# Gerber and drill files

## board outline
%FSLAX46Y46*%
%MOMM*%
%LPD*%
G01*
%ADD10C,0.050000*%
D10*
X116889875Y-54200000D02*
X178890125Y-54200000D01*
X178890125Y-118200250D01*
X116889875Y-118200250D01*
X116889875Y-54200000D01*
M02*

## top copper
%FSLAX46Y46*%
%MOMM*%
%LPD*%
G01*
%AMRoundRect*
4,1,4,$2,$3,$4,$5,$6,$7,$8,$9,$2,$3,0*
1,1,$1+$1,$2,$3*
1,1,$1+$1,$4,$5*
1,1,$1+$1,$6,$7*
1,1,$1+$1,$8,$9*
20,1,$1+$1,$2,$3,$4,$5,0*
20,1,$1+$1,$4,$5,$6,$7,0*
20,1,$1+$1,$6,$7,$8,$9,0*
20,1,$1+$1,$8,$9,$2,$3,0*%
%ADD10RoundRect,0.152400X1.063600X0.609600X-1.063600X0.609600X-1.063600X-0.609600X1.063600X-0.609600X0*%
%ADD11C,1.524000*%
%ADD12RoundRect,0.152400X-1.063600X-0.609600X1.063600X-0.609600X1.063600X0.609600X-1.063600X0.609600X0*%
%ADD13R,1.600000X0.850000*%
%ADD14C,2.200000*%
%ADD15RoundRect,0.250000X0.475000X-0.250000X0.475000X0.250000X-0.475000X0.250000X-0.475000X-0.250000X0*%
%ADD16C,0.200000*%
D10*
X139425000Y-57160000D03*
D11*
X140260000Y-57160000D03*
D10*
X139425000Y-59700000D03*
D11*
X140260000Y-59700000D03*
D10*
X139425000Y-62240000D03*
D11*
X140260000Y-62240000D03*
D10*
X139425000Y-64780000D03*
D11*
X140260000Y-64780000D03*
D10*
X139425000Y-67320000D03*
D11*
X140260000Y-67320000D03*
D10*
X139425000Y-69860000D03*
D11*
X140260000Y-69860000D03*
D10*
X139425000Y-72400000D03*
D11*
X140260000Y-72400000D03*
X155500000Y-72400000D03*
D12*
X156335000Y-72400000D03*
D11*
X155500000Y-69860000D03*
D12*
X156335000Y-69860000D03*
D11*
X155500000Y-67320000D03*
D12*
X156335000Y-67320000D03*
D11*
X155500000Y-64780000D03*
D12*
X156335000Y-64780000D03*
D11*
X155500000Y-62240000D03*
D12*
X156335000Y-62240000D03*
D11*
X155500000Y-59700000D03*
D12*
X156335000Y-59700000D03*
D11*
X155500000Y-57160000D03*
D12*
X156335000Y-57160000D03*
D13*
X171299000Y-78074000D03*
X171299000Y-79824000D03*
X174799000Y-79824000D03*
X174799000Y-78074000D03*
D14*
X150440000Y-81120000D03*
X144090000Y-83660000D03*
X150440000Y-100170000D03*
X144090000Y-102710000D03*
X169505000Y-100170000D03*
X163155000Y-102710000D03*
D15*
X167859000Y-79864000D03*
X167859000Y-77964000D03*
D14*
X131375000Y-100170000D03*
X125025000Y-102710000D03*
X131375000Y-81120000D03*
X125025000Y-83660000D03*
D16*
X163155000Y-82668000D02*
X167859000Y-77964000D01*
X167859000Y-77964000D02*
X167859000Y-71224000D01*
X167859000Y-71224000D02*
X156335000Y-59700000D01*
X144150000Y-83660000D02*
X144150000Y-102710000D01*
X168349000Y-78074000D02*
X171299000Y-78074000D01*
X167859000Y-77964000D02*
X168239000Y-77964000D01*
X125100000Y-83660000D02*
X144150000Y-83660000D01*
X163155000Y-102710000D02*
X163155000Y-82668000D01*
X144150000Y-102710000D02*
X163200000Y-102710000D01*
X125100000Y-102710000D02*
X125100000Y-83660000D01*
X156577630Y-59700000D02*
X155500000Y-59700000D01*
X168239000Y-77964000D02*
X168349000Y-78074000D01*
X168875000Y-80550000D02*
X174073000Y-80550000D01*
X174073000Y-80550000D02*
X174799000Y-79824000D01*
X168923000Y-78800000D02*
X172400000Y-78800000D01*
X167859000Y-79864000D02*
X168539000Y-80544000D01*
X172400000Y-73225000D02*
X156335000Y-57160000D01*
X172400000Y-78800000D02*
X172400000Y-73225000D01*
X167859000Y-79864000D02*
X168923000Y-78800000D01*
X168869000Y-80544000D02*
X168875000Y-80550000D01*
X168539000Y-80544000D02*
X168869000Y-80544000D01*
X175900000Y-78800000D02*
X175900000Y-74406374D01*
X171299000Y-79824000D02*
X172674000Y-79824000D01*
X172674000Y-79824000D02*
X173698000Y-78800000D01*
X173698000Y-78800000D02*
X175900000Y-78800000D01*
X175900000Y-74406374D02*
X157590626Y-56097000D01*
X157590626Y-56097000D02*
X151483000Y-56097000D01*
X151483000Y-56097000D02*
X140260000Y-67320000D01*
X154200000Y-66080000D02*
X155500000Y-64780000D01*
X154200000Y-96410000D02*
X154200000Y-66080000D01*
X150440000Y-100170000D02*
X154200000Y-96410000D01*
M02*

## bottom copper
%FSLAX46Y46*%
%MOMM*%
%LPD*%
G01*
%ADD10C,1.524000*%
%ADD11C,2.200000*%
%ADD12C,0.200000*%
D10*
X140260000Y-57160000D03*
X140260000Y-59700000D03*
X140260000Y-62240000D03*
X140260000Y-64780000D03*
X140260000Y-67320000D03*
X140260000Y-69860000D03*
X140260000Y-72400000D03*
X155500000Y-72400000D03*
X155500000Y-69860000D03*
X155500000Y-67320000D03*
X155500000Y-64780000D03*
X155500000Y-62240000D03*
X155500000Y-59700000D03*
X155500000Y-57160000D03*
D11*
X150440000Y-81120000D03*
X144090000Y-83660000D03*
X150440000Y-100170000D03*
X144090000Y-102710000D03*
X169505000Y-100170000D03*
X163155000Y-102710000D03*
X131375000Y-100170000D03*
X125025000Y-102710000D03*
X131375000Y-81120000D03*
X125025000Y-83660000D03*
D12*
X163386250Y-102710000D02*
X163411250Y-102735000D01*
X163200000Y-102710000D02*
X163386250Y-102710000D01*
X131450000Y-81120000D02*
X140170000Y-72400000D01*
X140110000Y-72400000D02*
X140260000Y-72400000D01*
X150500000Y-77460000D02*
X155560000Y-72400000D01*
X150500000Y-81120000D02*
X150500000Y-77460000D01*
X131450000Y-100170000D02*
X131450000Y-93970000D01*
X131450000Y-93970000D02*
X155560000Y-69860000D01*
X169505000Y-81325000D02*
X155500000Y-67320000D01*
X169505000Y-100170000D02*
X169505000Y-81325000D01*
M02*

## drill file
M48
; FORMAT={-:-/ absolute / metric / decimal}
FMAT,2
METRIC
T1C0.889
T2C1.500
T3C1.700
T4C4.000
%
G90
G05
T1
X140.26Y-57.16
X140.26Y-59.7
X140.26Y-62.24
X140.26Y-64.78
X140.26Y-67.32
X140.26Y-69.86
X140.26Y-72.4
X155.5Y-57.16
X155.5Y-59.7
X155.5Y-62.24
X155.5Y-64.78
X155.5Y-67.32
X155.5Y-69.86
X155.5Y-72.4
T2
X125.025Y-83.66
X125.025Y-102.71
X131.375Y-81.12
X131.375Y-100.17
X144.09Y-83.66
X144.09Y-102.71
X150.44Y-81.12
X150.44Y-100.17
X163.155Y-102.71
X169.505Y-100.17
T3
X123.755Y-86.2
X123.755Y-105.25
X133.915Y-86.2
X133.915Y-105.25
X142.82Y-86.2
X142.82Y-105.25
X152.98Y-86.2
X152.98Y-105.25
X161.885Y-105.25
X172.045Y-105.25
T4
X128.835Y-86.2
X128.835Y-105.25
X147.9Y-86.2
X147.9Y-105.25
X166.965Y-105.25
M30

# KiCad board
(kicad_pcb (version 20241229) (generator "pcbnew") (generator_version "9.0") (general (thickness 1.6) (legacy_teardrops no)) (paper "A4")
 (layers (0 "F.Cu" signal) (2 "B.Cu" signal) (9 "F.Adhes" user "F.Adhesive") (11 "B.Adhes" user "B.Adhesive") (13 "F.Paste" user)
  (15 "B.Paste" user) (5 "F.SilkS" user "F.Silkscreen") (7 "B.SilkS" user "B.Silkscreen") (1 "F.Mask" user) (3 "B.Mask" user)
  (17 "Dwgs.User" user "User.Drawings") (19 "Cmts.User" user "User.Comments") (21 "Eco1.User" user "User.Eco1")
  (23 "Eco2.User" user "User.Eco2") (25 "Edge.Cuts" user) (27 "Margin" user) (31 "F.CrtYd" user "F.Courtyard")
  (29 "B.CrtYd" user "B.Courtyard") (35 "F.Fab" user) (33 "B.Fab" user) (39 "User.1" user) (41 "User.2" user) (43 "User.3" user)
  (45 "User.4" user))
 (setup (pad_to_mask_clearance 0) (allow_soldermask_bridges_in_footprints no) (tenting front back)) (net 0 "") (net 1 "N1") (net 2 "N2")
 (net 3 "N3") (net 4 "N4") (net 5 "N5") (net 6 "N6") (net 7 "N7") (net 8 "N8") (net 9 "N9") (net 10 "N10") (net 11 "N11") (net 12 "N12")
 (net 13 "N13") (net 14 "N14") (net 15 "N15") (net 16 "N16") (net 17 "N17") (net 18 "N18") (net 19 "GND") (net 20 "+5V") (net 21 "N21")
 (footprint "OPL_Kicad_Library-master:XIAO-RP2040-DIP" (layer "F.Cu") (at 147.88 64.78)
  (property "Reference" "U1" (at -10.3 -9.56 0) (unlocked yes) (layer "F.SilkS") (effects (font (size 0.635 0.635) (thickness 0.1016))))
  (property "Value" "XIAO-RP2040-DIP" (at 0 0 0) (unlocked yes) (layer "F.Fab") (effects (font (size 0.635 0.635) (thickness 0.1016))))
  (pad "1" smd roundrect (at -8.455 -7.62 180) (size 2.432 1.524) (layers "F.Cu" "F.Mask") (roundrect_rratio 0.1) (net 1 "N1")
   (thermal_bridge_angle 45))
  (pad "1" thru_hole circle (at -7.62 -7.62 180) (size 1.524 1.524) (drill 0.889) (layers "*.Cu" "*.Mask") (remove_unused_layers no)
   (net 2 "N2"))
  (pad "2" smd roundrect (at -8.455 -5.08 180) (size 2.432 1.524) (layers "F.Cu" "F.Mask") (roundrect_rratio 0.1) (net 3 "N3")
   (thermal_bridge_angle 45))
  (pad "2" thru_hole circle (at -7.62 -5.08 180) (size 1.524 1.524) (drill 0.889) (layers "*.Cu" "*.Mask") (remove_unused_layers no)
   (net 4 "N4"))
  (pad "3" smd roundrect (at -8.455 -2.54 180) (size 2.432 1.524) (layers "F.Cu" "F.Mask") (roundrect_rratio 0.1) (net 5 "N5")
   (thermal_bridge_angle 45))
  (pad "3" thru_hole circle (at -7.62 -2.54 180) (size 1.524 1.524) (drill 0.889) (layers "*.Cu" "*.Mask") (remove_unused_layers no)
   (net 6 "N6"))
  (pad "4" smd roundrect (at -8.455 0 180) (size 2.432 1.524) (layers "F.Cu" "F.Mask") (roundrect_rratio 0.1) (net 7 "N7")
   (thermal_bridge_angle 45))
  (pad "4" thru_hole circle (at -7.62 0 180) (size 1.524 1.524) (drill 0.889) (layers "*.Cu" "*.Mask") (remove_unused_layers no)
   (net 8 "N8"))
  (pad "5" smd roundrect (at -8.455 2.54 180) (size 2.432 1.524) (layers "F.Cu" "F.Mask") (roundrect_rratio 0.1) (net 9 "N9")
   (thermal_bridge_angle 45))
  (pad "5" thru_hole circle (at -7.62 2.54 180) (size 1.524 1.524) (drill 0.889) (layers "*.Cu" "*.Mask") (remove_unused_layers no)
   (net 9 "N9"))
  (pad "6" smd roundrect (at -8.455 5.08 180) (size 2.432 1.524) (layers "F.Cu" "F.Mask") (roundrect_rratio 0.1) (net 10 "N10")
   (thermal_bridge_angle 45))
  (pad "6" thru_hole circle (at -7.62 5.08 180) (size 1.524 1.524) (drill 0.889) (layers "*.Cu" "*.Mask") (remove_unused_layers no)
   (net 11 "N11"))
  (pad "7" smd roundrect (at -8.455 7.62 180) (size 2.432 1.524) (layers "F.Cu" "F.Mask") (roundrect_rratio 0.1) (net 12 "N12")
   (thermal_bridge_angle 45))
  (pad "7" thru_hole circle (at -7.62 7.62 180) (size 1.524 1.524) (drill 0.889) (layers "*.Cu" "*.Mask") (remove_unused_layers no)
   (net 12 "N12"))
  (pad "8" thru_hole circle (at 7.62 7.62) (size 1.524 1.524) (drill 0.889) (layers "*.Cu" "*.Mask") (remove_unused_layers no)
   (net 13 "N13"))
  (pad "8" smd roundrect (at 8.455 7.62) (size 2.432 1.524) (layers "F.Cu" "F.Mask") (roundrect_rratio 0.1) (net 13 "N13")
   (thermal_bridge_angle 45))
  (pad "9" thru_hole circle (at 7.62 5.08) (size 1.524 1.524) (drill 0.889) (layers "*.Cu" "*.Mask") (remove_unused_layers no)
   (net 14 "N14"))
  (pad "9" smd roundrect (at 8.455 5.08) (size 2.432 1.524) (layers "F.Cu" "F.Mask") (roundrect_rratio 0.1) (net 14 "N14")
   (thermal_bridge_angle 45))
  (pad "10" thru_hole circle (at 7.62 2.54) (size 1.524 1.524) (drill 0.889) (layers "*.Cu" "*.Mask") (remove_unused_layers no)
   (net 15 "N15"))
  (pad "10" smd roundrect (at 8.455 2.54) (size 2.432 1.524) (layers "F.Cu" "F.Mask") (roundrect_rratio 0.1) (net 15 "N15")
   (thermal_bridge_angle 45))
  (pad "11" thru_hole circle (at 7.62 0) (size 1.524 1.524) (drill 0.889) (layers "*.Cu" "*.Mask") (remove_unused_layers no) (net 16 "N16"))
  (pad "11" smd roundrect (at 8.455 0) (size 2.432 1.524) (layers "F.Cu" "F.Mask") (roundrect_rratio 0.1) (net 16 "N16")
   (thermal_bridge_angle 45))
  (pad "12" thru_hole circle (at 7.62 -2.54) (size 1.524 1.524) (drill 0.889) (layers "*.Cu" "*.Mask") (remove_unused_layers no)
   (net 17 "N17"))
  (pad "12" smd roundrect (at 8.455 -2.54) (size 2.432 1.524) (layers "F.Cu" "F.Mask") (roundrect_rratio 0.1) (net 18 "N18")
   (thermal_bridge_angle 45))
  (pad "13" thru_hole circle (at 7.62 -5.08) (size 1.524 1.524) (drill 0.889) (layers "*.Cu" "*.Mask") (remove_unused_layers no)
   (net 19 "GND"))
  (pad "13" smd roundrect (at 8.455 -5.08) (size 2.432 1.524) (layers "F.Cu" "F.Mask") (roundrect_rratio 0.1) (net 19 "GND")
   (thermal_bridge_angle 45))
  (pad "14" thru_hole circle (at 7.62 -7.62) (size 1.524 1.524) (drill 0.889) (layers "*.Cu" "*.Mask") (remove_unused_layers no)
   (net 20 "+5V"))
  (pad "14" smd roundrect (at 8.455 -7.62) (size 2.432 1.524) (layers "F.Cu" "F.Mask") (roundrect_rratio 0.1) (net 20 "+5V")
   (thermal_bridge_angle 45)))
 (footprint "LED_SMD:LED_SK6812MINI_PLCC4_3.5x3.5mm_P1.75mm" (layer "F.Cu") (at 173.049 78.949)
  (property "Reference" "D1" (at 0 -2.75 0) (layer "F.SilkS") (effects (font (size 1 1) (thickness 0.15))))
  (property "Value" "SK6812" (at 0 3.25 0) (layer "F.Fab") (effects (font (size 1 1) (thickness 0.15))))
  (pad "1" smd rect (at -1.75 -0.875) (size 1.6 0.85) (layers "F.Cu" "F.Mask" "F.Paste") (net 19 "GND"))
  (pad "2" smd rect (at -1.75 0.875) (size 1.6 0.85) (layers "F.Cu" "F.Mask" "F.Paste") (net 9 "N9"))
  (pad "3" smd rect (at 1.75 0.875) (size 1.6 0.85) (layers "F.Cu" "F.Mask" "F.Paste") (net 20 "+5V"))
  (pad "4" smd rect (at 1.75 -0.875) (size 1.6 0.85) (layers "F.Cu" "F.Mask" "F.Paste") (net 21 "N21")))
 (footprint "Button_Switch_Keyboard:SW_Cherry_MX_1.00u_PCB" (layer "F.Cu") (at 150.44 81.12)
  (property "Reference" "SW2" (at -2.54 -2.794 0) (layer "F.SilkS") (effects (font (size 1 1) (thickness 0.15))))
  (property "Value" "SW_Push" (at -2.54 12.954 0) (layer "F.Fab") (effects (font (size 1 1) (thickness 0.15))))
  (pad "" np_thru_hole circle (at -7.62 5.08) (size 1.7 1.7) (drill 1.7) (layers "*.Cu" "*.Mask"))
  (pad "" np_thru_hole circle (at -2.54 5.08) (size 4 4) (drill 4) (layers "*.Cu" "*.Mask"))
  (pad "" np_thru_hole circle (at 2.54 5.08) (size 1.7 1.7) (drill 1.7) (layers "*.Cu" "*.Mask"))
  (pad "1" thru_hole circle (at 0 0) (size 2.2 2.2) (drill 1.5) (layers "*.Cu" "*.Mask") (remove_unused_layers no) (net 13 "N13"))
  (pad "2" thru_hole circle (at -6.35 2.54) (size 2.2 2.2) (drill 1.5) (layers "*.Cu" "*.Mask") (remove_unused_layers no) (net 19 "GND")))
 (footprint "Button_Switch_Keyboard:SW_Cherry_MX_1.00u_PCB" (layer "F.Cu") (at 150.44 100.17)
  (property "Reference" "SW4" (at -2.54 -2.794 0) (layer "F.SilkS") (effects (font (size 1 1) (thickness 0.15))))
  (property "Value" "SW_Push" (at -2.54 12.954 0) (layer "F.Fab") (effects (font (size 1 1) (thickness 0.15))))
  (pad "" np_thru_hole circle (at -7.62 5.08) (size 1.7 1.7) (drill 1.7) (layers "*.Cu" "*.Mask"))
  (pad "" np_thru_hole circle (at -2.54 5.08) (size 4 4) (drill 4) (layers "*.Cu" "*.Mask"))
  (pad "" np_thru_hole circle (at 2.54 5.08) (size 1.7 1.7) (drill 1.7) (layers "*.Cu" "*.Mask"))
  (pad "1" thru_hole circle (at 0 0) (size 2.2 2.2) (drill 1.5) (layers "*.Cu" "*.Mask") (remove_unused_layers no) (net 16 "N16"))
  (pad "2" thru_hole circle (at -6.35 2.54) (size 2.2 2.2) (drill 1.5) (layers "*.Cu" "*.Mask") (remove_unused_layers no) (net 19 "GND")))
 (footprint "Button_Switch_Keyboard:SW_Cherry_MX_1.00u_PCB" (layer "F.Cu") (at 169.505 100.17)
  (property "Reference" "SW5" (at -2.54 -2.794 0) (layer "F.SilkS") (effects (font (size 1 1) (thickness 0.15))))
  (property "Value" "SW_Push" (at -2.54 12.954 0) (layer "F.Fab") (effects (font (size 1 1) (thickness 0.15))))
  (pad "" np_thru_hole circle (at -7.62 5.08) (size 1.7 1.7) (drill 1.7) (layers "*.Cu" "*.Mask"))
  (pad "" np_thru_hole circle (at -2.54 5.08) (size 4 4) (drill 4) (layers "*.Cu" "*.Mask"))
  (pad "" np_thru_hole circle (at 2.54 5.08) (size 1.7 1.7) (drill 1.7) (layers "*.Cu" "*.Mask"))
  (pad "1" thru_hole circle (at 0 0) (size 2.2 2.2) (drill 1.5) (layers "*.Cu" "*.Mask") (remove_unused_layers no) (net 15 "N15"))
  (pad "2" thru_hole circle (at -6.35 2.54) (size 2.2 2.2) (drill 1.5) (layers "*.Cu" "*.Mask") (remove_unused_layers no) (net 19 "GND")))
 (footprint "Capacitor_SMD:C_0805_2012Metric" (layer "F.Cu") (at 167.859 78.914 90)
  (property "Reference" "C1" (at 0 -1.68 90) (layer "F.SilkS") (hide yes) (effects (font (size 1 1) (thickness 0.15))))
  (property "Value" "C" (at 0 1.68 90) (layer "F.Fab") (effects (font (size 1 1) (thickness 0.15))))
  (pad "1" smd roundrect (at -0.95 0 90) (size 1 1.45) (layers "F.Cu" "F.Mask" "F.Paste") (roundrect_rratio 0.25) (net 20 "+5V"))
  (pad "2" smd roundrect (at 0.95 0 90) (size 1 1.45) (layers "F.Cu" "F.Mask" "F.Paste") (roundrect_rratio 0.25) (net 19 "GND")))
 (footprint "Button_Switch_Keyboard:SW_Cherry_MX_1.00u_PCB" (layer "F.Cu") (at 131.375 100.17)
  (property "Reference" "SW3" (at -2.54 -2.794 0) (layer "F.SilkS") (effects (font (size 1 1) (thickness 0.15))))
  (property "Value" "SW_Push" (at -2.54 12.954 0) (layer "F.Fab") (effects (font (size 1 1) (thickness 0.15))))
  (pad "" np_thru_hole circle (at -7.62 5.08) (size 1.7 1.7) (drill 1.7) (layers "*.Cu" "*.Mask"))
  (pad "" np_thru_hole circle (at -2.54 5.08) (size 4 4) (drill 4) (layers "*.Cu" "*.Mask"))
  (pad "" np_thru_hole circle (at 2.54 5.08) (size 1.7 1.7) (drill 1.7) (layers "*.Cu" "*.Mask"))
  (pad "1" thru_hole circle (at 0 0) (size 2.2 2.2) (drill 1.5) (layers "*.Cu" "*.Mask") (remove_unused_layers no) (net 14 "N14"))
  (pad "2" thru_hole circle (at -6.35 2.54) (size 2.2 2.2) (drill 1.5) (layers "*.Cu" "*.Mask") (remove_unused_layers no) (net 19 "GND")))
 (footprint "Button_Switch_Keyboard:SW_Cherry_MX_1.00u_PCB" (layer "F.Cu") (at 131.375 81.12)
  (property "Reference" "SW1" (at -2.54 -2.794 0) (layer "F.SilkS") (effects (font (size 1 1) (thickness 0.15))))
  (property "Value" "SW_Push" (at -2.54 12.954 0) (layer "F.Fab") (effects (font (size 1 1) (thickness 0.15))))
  (pad "" np_thru_hole circle (at -7.62 5.08) (size 1.7 1.7) (drill 1.7) (layers "*.Cu" "*.Mask"))
  (pad "" np_thru_hole circle (at -2.54 5.08) (size 4 4) (drill 4) (layers "*.Cu" "*.Mask"))
  (pad "" np_thru_hole circle (at 2.54 5.08) (size 1.7 1.7) (drill 1.7) (layers "*.Cu" "*.Mask"))
  (pad "1" thru_hole circle (at 0 0) (size 2.2 2.2) (drill 1.5) (layers "*.Cu" "*.Mask") (remove_unused_layers no) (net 12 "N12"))
  (pad "2" thru_hole circle (at -6.35 2.54) (size 2.2 2.2) (drill 1.5) (layers "*.Cu" "*.Mask") (remove_unused_layers no) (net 19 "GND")))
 (gr_rect (start 116.889875 54.2) (end 178.890125 118.20025) (stroke (width 0.05) (type default)) (fill no) (layer "Edge.Cuts"))
 (segment (start 163.155 82.668) (end 167.859 77.964) (width 0.2) (layer "F.Cu") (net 19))
 (segment (start 167.859 77.964) (end 167.859 71.224) (width 0.2) (layer "F.Cu") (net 19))
 (segment (start 167.859 71.224) (end 156.335 59.7) (width 0.2) (layer "F.Cu") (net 19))
 (segment (start 144.15 83.66) (end 144.15 102.71) (width 0.2) (layer "F.Cu") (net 19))
 (segment (start 168.349 78.074) (end 171.299 78.074) (width 0.2) (layer "F.Cu") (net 19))
 (segment (start 167.859 77.964) (end 168.239 77.964) (width 0.2) (layer "F.Cu") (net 19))
 (segment (start 125.1 83.66) (end 144.15 83.66) (width 0.2) (layer "F.Cu") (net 19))
 (segment (start 163.155 102.71) (end 163.155 82.668) (width 0.2) (layer "F.Cu") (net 19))
 (segment (start 144.15 102.71) (end 163.2 102.71) (width 0.2) (layer "F.Cu") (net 19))
 (segment (start 125.1 102.71) (end 125.1 83.66) (width 0.2) (layer "F.Cu") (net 19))
 (segment (start 156.57763 59.7) (end 155.5 59.7) (width 0.2) (layer "F.Cu") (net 19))
 (segment (start 168.239 77.964) (end 168.349 78.074) (width 0.2) (layer "F.Cu") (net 19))
 (segment (start 163.38625 102.71) (end 163.41125 102.735) (width 0.2) (layer "B.Cu") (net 19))
 (segment (start 163.2 102.71) (end 163.38625 102.71) (width 0.2) (layer "B.Cu") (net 19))
 (segment (start 168.875 80.55) (end 174.073 80.55) (width 0.2) (layer "F.Cu") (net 20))
 (segment (start 174.073 80.55) (end 174.799 79.824) (width 0.2) (layer "F.Cu") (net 20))
 (segment (start 168.923 78.8) (end 172.4 78.8) (width 0.2) (layer "F.Cu") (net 20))
 (segment (start 167.859 79.864) (end 168.539 80.544) (width 0.2) (layer "F.Cu") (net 20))
 (segment (start 172.4 73.225) (end 156.335 57.16) (width 0.2) (layer "F.Cu") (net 20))
 (segment (start 172.4 78.8) (end 172.4 73.225) (width 0.2) (layer "F.Cu") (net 20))
 (segment (start 167.859 79.864) (end 168.923 78.8) (width 0.2) (layer "F.Cu") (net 20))
 (segment (start 168.869 80.544) (end 168.875 80.55) (width 0.2) (layer "F.Cu") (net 20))
 (segment (start 168.539 80.544) (end 168.869 80.544) (width 0.2) (layer "F.Cu") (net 20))
 (segment (start 175.9 78.8) (end 175.9 74.406374) (width 0.2) (layer "F.Cu") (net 9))
 (segment (start 171.299 79.824) (end 172.674 79.824) (width 0.2) (layer "F.Cu") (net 9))
 (segment (start 172.674 79.824) (end 173.698 78.8) (width 0.2) (layer "F.Cu") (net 9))
 (segment (start 173.698 78.8) (end 175.9 78.8) (width 0.2) (layer "F.Cu") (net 9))
 (segment (start 175.9 74.406374) (end 157.590626 56.097) (width 0.2) (layer "F.Cu") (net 9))
 (segment (start 157.590626 56.097) (end 151.483 56.097) (width 0.2) (layer "F.Cu") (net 9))
 (segment (start 151.483 56.097) (end 140.26 67.32) (width 0.2) (layer "F.Cu") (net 9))
 (segment (start 131.45 81.12) (end 140.17 72.4) (width 0.2) (layer "B.Cu") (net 12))
 (segment (start 140.11 72.4) (end 140.26 72.4) (width 0.2) (layer "B.Cu") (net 12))
 (segment (start 150.5 77.46) (end 155.56 72.4) (width 0.2) (layer "B.Cu") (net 13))
 (segment (start 150.5 81.12) (end 150.5 77.46) (width 0.2) (layer "B.Cu") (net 13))
 (segment (start 131.45 100.17) (end 131.45 93.97) (width 0.2) (layer "B.Cu") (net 14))
 (segment (start 131.45 93.97) (end 155.56 69.86) (width 0.2) (layer "B.Cu") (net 14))
 (segment (start 154.2 66.08) (end 155.5 64.78) (width 0.2) (layer "F.Cu") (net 16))
 (segment (start 154.2 96.41) (end 154.2 66.08) (width 0.2) (layer "F.Cu") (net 16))
 (segment (start 150.44 100.17) (end 154.2 96.41) (width 0.2) (layer "F.Cu") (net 16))
 (segment (start 169.505 81.325) (end 155.5 67.32) (width 0.2) (layer "B.Cu") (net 15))
 (segment (start 169.505 100.17) (end 169.505 81.325) (width 0.2) (layer "B.Cu") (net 15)))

